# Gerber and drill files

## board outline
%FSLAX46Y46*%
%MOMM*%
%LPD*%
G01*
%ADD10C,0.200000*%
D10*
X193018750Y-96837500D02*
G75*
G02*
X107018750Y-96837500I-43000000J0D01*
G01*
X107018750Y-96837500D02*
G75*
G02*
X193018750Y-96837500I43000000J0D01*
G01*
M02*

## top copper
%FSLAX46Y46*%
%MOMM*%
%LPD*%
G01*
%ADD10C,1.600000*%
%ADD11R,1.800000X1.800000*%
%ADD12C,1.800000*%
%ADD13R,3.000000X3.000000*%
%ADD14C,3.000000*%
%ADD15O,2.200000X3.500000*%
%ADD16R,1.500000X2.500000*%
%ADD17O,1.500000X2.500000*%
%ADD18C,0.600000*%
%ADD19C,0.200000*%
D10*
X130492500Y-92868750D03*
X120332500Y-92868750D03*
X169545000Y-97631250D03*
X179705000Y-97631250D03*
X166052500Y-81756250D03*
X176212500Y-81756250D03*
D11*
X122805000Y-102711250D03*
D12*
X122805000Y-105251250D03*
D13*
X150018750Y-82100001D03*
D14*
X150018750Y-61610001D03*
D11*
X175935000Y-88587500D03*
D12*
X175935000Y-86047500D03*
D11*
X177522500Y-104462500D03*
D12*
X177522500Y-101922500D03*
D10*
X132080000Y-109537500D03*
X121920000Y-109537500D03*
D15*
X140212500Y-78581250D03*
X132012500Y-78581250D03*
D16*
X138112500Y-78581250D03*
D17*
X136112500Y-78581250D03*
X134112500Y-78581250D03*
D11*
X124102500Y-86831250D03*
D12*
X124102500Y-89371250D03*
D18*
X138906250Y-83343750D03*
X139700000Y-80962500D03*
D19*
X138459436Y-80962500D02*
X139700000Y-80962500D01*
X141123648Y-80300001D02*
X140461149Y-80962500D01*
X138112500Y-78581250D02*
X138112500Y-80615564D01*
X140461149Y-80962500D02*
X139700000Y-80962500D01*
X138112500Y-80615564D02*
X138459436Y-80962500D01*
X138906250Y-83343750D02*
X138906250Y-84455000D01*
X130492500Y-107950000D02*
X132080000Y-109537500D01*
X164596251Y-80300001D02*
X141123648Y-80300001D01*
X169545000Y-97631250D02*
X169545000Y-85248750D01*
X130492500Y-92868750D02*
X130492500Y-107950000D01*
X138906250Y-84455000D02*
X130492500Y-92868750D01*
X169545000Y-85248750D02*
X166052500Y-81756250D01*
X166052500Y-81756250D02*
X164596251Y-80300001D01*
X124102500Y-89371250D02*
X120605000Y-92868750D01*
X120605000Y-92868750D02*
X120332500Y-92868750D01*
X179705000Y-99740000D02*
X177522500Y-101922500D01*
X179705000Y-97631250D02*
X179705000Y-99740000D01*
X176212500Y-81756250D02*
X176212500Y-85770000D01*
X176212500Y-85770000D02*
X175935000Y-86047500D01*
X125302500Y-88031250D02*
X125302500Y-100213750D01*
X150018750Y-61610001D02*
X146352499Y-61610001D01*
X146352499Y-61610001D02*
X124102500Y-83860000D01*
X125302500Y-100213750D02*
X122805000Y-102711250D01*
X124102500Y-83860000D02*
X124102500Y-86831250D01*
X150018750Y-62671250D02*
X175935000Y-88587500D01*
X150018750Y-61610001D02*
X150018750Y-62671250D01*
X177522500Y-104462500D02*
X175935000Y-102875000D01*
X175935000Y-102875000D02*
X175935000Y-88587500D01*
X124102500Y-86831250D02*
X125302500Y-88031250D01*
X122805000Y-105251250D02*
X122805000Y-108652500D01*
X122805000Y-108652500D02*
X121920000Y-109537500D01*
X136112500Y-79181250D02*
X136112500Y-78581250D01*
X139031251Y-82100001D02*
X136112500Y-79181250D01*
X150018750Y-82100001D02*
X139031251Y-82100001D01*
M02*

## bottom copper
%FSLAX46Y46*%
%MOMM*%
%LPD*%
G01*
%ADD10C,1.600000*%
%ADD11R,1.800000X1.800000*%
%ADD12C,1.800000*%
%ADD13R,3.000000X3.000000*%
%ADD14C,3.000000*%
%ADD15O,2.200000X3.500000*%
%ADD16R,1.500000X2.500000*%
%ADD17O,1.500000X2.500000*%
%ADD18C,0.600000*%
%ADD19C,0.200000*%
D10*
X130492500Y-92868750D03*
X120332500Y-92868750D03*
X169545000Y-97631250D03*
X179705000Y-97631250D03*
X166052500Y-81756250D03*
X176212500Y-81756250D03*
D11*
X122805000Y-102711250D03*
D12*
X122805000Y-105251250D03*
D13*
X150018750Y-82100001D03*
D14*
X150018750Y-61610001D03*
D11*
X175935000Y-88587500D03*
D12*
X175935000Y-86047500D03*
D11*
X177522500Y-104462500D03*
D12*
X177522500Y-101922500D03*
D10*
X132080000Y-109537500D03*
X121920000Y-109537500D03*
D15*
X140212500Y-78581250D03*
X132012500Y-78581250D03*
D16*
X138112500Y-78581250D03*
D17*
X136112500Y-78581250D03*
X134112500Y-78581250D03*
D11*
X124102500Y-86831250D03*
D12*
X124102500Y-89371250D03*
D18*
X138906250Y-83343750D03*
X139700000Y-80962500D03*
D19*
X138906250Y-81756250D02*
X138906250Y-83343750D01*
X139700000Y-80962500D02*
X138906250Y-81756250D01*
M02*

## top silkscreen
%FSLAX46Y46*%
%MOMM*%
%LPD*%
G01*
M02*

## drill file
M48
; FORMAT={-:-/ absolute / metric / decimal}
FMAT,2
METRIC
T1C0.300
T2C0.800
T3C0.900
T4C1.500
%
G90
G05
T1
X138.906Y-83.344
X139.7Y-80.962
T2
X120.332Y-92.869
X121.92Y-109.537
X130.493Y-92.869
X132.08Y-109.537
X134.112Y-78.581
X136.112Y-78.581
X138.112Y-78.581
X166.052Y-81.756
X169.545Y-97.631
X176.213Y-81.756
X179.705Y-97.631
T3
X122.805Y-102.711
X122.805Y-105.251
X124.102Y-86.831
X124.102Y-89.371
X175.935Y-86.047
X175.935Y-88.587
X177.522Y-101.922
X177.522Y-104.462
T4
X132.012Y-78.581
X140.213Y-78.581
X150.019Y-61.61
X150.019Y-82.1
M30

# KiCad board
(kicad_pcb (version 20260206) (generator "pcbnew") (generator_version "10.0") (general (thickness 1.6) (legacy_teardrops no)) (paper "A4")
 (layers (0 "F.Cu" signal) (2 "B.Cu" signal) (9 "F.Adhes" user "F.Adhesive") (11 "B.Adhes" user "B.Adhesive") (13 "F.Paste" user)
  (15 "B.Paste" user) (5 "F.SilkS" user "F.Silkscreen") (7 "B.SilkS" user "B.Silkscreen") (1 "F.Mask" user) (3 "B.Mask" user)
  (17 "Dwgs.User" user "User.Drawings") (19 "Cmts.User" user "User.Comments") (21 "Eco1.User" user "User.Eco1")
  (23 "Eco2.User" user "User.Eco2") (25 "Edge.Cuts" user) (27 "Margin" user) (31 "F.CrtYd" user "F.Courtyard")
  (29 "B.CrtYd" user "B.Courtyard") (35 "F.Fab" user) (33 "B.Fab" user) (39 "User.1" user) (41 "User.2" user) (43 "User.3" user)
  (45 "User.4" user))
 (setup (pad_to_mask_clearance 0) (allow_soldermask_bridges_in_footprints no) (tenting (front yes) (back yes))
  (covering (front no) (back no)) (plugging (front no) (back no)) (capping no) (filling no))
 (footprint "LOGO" (layer "F.Cu") (at 150.01875 96.8375)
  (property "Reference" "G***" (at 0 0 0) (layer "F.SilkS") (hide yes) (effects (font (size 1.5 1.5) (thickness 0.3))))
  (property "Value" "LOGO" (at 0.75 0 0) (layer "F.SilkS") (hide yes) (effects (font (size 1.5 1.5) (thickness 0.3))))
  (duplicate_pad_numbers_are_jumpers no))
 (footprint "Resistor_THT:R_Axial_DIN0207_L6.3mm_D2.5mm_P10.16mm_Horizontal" (layer "B.Cu") (at 130.4925 92.86875 180)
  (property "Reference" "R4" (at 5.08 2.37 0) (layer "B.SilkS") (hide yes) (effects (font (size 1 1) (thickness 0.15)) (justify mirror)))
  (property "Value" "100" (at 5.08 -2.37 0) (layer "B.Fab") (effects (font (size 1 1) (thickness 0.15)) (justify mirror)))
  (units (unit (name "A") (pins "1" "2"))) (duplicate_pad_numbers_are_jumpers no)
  (pad "1" thru_hole circle (at 0 0 180) (size 1.6 1.6) (drill 0.8) (layers "*.Cu" "*.Mask") (remove_unused_layers no) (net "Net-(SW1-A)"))
  (pad "2" thru_hole circle (at 10.16 0 180) (size 1.6 1.6) (drill 0.8) (layers "*.Cu" "*.Mask") (remove_unused_layers no)
   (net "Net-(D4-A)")))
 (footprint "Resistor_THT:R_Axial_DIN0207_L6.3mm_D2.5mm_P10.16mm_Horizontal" (layer "B.Cu") (at 169.545 97.63125)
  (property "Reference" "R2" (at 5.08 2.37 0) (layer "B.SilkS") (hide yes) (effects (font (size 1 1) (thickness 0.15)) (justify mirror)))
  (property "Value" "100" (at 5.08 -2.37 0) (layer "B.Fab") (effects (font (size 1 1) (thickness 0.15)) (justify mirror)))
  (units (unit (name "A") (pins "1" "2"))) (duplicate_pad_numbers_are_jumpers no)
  (pad "1" thru_hole circle (at 0 0) (size 1.6 1.6) (drill 0.8) (layers "*.Cu" "*.Mask") (remove_unused_layers no) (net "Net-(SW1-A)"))
  (pad "2" thru_hole circle (at 10.16 0) (size 1.6 1.6) (drill 0.8) (layers "*.Cu" "*.Mask") (remove_unused_layers no) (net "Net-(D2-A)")))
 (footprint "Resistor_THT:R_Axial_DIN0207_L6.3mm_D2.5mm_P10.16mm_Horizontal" (layer "B.Cu") (at 166.0525 81.75625)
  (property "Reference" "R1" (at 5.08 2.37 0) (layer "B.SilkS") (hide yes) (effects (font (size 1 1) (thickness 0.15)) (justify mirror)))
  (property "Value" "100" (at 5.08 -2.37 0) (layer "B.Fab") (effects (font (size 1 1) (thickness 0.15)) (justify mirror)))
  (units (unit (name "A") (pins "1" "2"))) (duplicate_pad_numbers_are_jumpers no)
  (pad "1" thru_hole circle (at 0 0) (size 1.6 1.6) (drill 0.8) (layers "*.Cu" "*.Mask") (remove_unused_layers no) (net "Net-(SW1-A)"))
  (pad "2" thru_hole circle (at 10.16 0) (size 1.6 1.6) (drill 0.8) (layers "*.Cu" "*.Mask") (remove_unused_layers no) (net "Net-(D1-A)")))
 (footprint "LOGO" (layer "B.Cu") (at 150.01875 96.8375 180)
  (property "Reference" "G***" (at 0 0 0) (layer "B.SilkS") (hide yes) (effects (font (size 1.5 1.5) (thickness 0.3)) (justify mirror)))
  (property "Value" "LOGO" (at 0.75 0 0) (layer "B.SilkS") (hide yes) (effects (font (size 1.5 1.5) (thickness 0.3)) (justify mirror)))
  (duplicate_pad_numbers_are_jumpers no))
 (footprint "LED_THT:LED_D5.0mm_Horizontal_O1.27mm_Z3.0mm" (layer "B.Cu") (at 122.805 102.71125 -90)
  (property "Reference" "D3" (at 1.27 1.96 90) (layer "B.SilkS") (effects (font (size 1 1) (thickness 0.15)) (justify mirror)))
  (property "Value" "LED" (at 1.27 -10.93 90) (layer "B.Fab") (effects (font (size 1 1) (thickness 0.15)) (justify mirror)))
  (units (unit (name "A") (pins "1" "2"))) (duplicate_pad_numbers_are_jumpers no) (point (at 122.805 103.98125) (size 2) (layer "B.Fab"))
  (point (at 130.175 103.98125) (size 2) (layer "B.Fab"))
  (pad "1" thru_hole rect (at 0 0 270) (size 1.8 1.8) (drill 0.9) (layers "*.Cu" "*.Mask") (remove_unused_layers no) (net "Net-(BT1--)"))
  (pad "2" thru_hole circle (at 2.54 0 270) (size 1.8 1.8) (drill 0.9) (layers "*.Cu" "*.Mask") (remove_unused_layers no) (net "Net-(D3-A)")))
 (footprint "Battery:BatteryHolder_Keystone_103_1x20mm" (layer "B.Cu") (at 150.01875 82.100001 90)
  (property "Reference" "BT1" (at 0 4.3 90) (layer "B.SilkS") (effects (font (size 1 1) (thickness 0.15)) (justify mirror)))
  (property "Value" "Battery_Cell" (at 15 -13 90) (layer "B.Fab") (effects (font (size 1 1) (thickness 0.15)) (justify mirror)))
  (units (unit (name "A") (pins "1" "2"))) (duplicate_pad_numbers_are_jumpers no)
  (pad "1" thru_hole rect (at 0 0 90) (size 3 3) (drill 1.5) (layers "*.Cu" "*.Mask") (remove_unused_layers no) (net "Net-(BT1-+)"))
  (pad "2" thru_hole circle (at 20.49 0 90) (size 3 3) (drill 1.5) (layers "*.Cu" "*.Mask") (remove_unused_layers no) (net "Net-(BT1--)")))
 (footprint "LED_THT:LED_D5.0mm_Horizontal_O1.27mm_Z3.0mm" (layer "B.Cu") (at 175.935 88.5875 90)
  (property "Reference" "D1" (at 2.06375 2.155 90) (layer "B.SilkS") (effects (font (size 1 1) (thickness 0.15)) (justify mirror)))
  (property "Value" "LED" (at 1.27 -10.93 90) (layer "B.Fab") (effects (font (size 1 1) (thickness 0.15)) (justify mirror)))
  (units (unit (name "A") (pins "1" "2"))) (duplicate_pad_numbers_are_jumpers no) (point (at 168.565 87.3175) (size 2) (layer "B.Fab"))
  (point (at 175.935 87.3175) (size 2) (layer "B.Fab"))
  (pad "1" thru_hole rect (at 0 0 90) (size 1.8 1.8) (drill 0.9) (layers "*.Cu" "*.Mask") (remove_unused_layers no) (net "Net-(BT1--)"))
  (pad "2" thru_hole circle (at 2.54 0 90) (size 1.8 1.8) (drill 0.9) (layers "*.Cu" "*.Mask") (remove_unused_layers no) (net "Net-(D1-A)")))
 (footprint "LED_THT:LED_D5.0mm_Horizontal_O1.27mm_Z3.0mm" (layer "B.Cu") (at 177.5225 104.4625 90)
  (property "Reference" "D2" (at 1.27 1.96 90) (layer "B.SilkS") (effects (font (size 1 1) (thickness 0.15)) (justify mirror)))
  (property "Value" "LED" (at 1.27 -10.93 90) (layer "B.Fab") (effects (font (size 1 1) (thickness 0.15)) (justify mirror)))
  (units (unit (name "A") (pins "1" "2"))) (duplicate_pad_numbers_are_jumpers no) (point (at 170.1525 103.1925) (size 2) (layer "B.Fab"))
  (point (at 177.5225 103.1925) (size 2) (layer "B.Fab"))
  (pad "1" thru_hole rect (at 0 0 90) (size 1.8 1.8) (drill 0.9) (layers "*.Cu" "*.Mask") (remove_unused_layers no) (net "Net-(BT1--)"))
  (pad "2" thru_hole circle (at 2.54 0 90) (size 1.8 1.8) (drill 0.9) (layers "*.Cu" "*.Mask") (remove_unused_layers no) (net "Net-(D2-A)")))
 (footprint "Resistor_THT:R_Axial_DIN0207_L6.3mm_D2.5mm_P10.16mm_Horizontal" (layer "B.Cu") (at 132.08 109.5375 180)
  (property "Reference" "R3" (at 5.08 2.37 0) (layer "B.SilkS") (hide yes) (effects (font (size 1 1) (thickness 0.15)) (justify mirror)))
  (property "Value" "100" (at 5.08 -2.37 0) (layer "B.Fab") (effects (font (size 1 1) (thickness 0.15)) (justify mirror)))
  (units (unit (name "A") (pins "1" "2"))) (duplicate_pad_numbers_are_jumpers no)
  (pad "1" thru_hole circle (at 0 0 180) (size 1.6 1.6) (drill 0.8) (layers "*.Cu" "*.Mask") (remove_unused_layers no) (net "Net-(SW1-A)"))
  (pad "2" thru_hole circle (at 10.16 0 180) (size 1.6 1.6) (drill 0.8) (layers "*.Cu" "*.Mask") (remove_unused_layers no)
   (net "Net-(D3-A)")))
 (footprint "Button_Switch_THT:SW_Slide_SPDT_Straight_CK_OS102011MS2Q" (layer "B.Cu") (at 138.1125 78.58125 180)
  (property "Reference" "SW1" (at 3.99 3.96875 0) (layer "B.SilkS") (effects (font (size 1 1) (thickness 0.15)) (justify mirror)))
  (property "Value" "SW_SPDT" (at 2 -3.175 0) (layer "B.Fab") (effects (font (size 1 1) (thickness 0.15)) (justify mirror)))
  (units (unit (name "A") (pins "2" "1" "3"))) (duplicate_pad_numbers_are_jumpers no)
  (pad "" thru_hole oval (at -2.1 0 180) (size 2.2 3.5) (drill 1.5) (layers "*.Cu" "*.Mask") (remove_unused_layers no))
  (pad "" thru_hole oval (at 6.1 0 180) (size 2.2 3.5) (drill 1.5) (layers "*.Cu" "*.Mask") (remove_unused_layers no))
  (pad "1" thru_hole rect (at 0 0 180) (size 1.5 2.5) (drill 0.8) (layers "*.Cu" "*.Mask") (remove_unused_layers no) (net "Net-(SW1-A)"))
  (pad "2" thru_hole oval (at 2 0 180) (size 1.5 2.5) (drill 0.8) (layers "*.Cu" "*.Mask") (remove_unused_layers no) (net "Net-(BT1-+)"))
  (pad "3" thru_hole oval (at 4 0 180) (size 1.5 2.5) (drill 0.8) (layers "*.Cu" "*.Mask") (remove_unused_layers no)
   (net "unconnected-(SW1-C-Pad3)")))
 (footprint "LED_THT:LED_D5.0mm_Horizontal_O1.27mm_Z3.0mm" (layer "B.Cu") (at 124.1025 86.83125 -90)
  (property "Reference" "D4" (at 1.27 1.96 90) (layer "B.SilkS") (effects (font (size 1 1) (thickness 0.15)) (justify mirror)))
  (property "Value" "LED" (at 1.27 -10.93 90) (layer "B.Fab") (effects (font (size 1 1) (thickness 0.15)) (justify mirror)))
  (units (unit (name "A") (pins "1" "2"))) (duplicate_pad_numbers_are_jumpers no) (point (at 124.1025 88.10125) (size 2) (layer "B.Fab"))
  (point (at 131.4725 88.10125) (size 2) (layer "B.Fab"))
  (pad "1" thru_hole rect (at 0 0 270) (size 1.8 1.8) (drill 0.9) (layers "*.Cu" "*.Mask") (remove_unused_layers no) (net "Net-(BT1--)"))
  (pad "2" thru_hole circle (at 2.54 0 270) (size 1.8 1.8) (drill 0.9) (layers "*.Cu" "*.Mask") (remove_unused_layers no) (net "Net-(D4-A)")))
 (gr_circle (center 150.01875 96.8375) (end 193.01875 96.8375) (stroke (width 0.2) (type default)) (fill no) (layer "Edge.Cuts"))
 (segment (start 138.459436 80.9625) (end 139.7 80.9625) (width 0.2) (layer "F.Cu") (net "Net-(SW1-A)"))
 (segment (start 141.123648 80.300001) (end 140.461149 80.9625) (width 0.2) (layer "F.Cu") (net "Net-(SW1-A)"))
 (segment (start 138.1125 78.58125) (end 138.1125 80.615564) (width 0.2) (layer "F.Cu") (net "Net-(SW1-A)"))
 (segment (start 140.461149 80.9625) (end 139.7 80.9625) (width 0.2) (layer "F.Cu") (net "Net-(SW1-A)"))
 (segment (start 138.1125 80.615564) (end 138.459436 80.9625) (width 0.2) (layer "F.Cu") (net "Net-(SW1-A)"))
 (segment (start 138.90625 83.34375) (end 138.90625 84.455) (width 0.2) (layer "F.Cu") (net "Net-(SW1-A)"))
 (segment (start 130.4925 107.95) (end 132.08 109.5375) (width 0.2) (layer "F.Cu") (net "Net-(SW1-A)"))
 (segment (start 164.596251 80.300001) (end 141.123648 80.300001) (width 0.2) (layer "F.Cu") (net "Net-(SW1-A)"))
 (segment (start 169.545 97.63125) (end 169.545 85.24875) (width 0.2) (layer "F.Cu") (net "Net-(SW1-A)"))
 (segment (start 130.4925 92.86875) (end 130.4925 107.95) (width 0.2) (layer "F.Cu") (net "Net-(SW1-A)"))
 (segment (start 138.90625 84.455) (end 130.4925 92.86875) (width 0.2) (layer "F.Cu") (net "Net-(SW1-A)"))
 (segment (start 169.545 85.24875) (end 166.0525 81.75625) (width 0.2) (layer "F.Cu") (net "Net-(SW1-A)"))
 (segment (start 166.0525 81.75625) (end 164.596251 80.300001) (width 0.2) (layer "F.Cu") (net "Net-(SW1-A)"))
 (via (at 138.90625 83.34375) (size 0.6) (drill 0.3) (layers "F.Cu" "B.Cu") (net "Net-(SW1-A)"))
 (via (at 139.7 80.9625) (size 0.6) (drill 0.3) (layers "F.Cu" "B.Cu") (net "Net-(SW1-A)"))
 (segment (start 138.90625 81.75625) (end 138.90625 83.34375) (width 0.2) (layer "B.Cu") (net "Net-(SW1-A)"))
 (segment (start 139.7 80.9625) (end 138.90625 81.75625) (width 0.2) (layer "B.Cu") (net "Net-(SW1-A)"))
 (segment (start 124.1025 89.37125) (end 120.605 92.86875) (width 0.2) (layer "F.Cu") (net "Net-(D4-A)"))
 (segment (start 120.605 92.86875) (end 120.3325 92.86875) (width 0.2) (layer "F.Cu") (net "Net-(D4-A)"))
 (segment (start 179.705 99.74) (end 177.5225 101.9225) (width 0.2) (layer "F.Cu") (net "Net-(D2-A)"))
 (segment (start 179.705 97.63125) (end 179.705 99.74) (width 0.2) (layer "F.Cu") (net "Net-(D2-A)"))
 (segment (start 176.2125 81.75625) (end 176.2125 85.77) (width 0.2) (layer "F.Cu") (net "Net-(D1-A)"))
 (segment (start 176.2125 85.77) (end 175.935 86.0475) (width 0.2) (layer "F.Cu") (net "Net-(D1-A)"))
 (segment (start 125.3025 88.03125) (end 125.3025 100.21375) (width 0.2) (layer "F.Cu") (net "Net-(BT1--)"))
 (segment (start 150.01875 61.610001) (end 146.352499 61.610001) (width 0.2) (layer "F.Cu") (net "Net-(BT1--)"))
 (segment (start 146.352499 61.610001) (end 124.1025 83.86) (width 0.2) (layer "F.Cu") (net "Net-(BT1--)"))
 (segment (start 125.3025 100.21375) (end 122.805 102.71125) (width 0.2) (layer "F.Cu") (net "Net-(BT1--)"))
 (segment (start 124.1025 83.86) (end 124.1025 86.83125) (width 0.2) (layer "F.Cu") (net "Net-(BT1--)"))
 (segment (start 150.01875 62.67125) (end 175.935 88.5875) (width 0.2) (layer "F.Cu") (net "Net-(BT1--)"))
 (segment (start 150.01875 61.610001) (end 150.01875 62.67125) (width 0.2) (layer "F.Cu") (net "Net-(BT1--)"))
 (segment (start 177.5225 104.4625) (end 175.935 102.875) (width 0.2) (layer "F.Cu") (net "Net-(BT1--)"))
 (segment (start 175.935 102.875) (end 175.935 88.5875) (width 0.2) (layer "F.Cu") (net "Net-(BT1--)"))
 (segment (start 124.1025 86.83125) (end 125.3025 88.03125) (width 0.2) (layer "F.Cu") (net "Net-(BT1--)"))
 (segment (start 122.805 105.25125) (end 122.805 108.6525) (width 0.2) (layer "F.Cu") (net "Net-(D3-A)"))
 (segment (start 122.805 108.6525) (end 121.92 109.5375) (width 0.2) (layer "F.Cu") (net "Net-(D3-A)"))
 (segment (start 136.1125 79.18125) (end 136.1125 78.58125) (width 0.2) (layer "F.Cu") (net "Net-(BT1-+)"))
 (segment (start 139.031251 82.100001) (end 136.1125 79.18125) (width 0.2) (layer "F.Cu") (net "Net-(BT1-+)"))
 (segment (start 150.01875 82.100001) (end 139.031251 82.100001) (width 0.2) (layer "F.Cu") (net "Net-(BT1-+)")))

